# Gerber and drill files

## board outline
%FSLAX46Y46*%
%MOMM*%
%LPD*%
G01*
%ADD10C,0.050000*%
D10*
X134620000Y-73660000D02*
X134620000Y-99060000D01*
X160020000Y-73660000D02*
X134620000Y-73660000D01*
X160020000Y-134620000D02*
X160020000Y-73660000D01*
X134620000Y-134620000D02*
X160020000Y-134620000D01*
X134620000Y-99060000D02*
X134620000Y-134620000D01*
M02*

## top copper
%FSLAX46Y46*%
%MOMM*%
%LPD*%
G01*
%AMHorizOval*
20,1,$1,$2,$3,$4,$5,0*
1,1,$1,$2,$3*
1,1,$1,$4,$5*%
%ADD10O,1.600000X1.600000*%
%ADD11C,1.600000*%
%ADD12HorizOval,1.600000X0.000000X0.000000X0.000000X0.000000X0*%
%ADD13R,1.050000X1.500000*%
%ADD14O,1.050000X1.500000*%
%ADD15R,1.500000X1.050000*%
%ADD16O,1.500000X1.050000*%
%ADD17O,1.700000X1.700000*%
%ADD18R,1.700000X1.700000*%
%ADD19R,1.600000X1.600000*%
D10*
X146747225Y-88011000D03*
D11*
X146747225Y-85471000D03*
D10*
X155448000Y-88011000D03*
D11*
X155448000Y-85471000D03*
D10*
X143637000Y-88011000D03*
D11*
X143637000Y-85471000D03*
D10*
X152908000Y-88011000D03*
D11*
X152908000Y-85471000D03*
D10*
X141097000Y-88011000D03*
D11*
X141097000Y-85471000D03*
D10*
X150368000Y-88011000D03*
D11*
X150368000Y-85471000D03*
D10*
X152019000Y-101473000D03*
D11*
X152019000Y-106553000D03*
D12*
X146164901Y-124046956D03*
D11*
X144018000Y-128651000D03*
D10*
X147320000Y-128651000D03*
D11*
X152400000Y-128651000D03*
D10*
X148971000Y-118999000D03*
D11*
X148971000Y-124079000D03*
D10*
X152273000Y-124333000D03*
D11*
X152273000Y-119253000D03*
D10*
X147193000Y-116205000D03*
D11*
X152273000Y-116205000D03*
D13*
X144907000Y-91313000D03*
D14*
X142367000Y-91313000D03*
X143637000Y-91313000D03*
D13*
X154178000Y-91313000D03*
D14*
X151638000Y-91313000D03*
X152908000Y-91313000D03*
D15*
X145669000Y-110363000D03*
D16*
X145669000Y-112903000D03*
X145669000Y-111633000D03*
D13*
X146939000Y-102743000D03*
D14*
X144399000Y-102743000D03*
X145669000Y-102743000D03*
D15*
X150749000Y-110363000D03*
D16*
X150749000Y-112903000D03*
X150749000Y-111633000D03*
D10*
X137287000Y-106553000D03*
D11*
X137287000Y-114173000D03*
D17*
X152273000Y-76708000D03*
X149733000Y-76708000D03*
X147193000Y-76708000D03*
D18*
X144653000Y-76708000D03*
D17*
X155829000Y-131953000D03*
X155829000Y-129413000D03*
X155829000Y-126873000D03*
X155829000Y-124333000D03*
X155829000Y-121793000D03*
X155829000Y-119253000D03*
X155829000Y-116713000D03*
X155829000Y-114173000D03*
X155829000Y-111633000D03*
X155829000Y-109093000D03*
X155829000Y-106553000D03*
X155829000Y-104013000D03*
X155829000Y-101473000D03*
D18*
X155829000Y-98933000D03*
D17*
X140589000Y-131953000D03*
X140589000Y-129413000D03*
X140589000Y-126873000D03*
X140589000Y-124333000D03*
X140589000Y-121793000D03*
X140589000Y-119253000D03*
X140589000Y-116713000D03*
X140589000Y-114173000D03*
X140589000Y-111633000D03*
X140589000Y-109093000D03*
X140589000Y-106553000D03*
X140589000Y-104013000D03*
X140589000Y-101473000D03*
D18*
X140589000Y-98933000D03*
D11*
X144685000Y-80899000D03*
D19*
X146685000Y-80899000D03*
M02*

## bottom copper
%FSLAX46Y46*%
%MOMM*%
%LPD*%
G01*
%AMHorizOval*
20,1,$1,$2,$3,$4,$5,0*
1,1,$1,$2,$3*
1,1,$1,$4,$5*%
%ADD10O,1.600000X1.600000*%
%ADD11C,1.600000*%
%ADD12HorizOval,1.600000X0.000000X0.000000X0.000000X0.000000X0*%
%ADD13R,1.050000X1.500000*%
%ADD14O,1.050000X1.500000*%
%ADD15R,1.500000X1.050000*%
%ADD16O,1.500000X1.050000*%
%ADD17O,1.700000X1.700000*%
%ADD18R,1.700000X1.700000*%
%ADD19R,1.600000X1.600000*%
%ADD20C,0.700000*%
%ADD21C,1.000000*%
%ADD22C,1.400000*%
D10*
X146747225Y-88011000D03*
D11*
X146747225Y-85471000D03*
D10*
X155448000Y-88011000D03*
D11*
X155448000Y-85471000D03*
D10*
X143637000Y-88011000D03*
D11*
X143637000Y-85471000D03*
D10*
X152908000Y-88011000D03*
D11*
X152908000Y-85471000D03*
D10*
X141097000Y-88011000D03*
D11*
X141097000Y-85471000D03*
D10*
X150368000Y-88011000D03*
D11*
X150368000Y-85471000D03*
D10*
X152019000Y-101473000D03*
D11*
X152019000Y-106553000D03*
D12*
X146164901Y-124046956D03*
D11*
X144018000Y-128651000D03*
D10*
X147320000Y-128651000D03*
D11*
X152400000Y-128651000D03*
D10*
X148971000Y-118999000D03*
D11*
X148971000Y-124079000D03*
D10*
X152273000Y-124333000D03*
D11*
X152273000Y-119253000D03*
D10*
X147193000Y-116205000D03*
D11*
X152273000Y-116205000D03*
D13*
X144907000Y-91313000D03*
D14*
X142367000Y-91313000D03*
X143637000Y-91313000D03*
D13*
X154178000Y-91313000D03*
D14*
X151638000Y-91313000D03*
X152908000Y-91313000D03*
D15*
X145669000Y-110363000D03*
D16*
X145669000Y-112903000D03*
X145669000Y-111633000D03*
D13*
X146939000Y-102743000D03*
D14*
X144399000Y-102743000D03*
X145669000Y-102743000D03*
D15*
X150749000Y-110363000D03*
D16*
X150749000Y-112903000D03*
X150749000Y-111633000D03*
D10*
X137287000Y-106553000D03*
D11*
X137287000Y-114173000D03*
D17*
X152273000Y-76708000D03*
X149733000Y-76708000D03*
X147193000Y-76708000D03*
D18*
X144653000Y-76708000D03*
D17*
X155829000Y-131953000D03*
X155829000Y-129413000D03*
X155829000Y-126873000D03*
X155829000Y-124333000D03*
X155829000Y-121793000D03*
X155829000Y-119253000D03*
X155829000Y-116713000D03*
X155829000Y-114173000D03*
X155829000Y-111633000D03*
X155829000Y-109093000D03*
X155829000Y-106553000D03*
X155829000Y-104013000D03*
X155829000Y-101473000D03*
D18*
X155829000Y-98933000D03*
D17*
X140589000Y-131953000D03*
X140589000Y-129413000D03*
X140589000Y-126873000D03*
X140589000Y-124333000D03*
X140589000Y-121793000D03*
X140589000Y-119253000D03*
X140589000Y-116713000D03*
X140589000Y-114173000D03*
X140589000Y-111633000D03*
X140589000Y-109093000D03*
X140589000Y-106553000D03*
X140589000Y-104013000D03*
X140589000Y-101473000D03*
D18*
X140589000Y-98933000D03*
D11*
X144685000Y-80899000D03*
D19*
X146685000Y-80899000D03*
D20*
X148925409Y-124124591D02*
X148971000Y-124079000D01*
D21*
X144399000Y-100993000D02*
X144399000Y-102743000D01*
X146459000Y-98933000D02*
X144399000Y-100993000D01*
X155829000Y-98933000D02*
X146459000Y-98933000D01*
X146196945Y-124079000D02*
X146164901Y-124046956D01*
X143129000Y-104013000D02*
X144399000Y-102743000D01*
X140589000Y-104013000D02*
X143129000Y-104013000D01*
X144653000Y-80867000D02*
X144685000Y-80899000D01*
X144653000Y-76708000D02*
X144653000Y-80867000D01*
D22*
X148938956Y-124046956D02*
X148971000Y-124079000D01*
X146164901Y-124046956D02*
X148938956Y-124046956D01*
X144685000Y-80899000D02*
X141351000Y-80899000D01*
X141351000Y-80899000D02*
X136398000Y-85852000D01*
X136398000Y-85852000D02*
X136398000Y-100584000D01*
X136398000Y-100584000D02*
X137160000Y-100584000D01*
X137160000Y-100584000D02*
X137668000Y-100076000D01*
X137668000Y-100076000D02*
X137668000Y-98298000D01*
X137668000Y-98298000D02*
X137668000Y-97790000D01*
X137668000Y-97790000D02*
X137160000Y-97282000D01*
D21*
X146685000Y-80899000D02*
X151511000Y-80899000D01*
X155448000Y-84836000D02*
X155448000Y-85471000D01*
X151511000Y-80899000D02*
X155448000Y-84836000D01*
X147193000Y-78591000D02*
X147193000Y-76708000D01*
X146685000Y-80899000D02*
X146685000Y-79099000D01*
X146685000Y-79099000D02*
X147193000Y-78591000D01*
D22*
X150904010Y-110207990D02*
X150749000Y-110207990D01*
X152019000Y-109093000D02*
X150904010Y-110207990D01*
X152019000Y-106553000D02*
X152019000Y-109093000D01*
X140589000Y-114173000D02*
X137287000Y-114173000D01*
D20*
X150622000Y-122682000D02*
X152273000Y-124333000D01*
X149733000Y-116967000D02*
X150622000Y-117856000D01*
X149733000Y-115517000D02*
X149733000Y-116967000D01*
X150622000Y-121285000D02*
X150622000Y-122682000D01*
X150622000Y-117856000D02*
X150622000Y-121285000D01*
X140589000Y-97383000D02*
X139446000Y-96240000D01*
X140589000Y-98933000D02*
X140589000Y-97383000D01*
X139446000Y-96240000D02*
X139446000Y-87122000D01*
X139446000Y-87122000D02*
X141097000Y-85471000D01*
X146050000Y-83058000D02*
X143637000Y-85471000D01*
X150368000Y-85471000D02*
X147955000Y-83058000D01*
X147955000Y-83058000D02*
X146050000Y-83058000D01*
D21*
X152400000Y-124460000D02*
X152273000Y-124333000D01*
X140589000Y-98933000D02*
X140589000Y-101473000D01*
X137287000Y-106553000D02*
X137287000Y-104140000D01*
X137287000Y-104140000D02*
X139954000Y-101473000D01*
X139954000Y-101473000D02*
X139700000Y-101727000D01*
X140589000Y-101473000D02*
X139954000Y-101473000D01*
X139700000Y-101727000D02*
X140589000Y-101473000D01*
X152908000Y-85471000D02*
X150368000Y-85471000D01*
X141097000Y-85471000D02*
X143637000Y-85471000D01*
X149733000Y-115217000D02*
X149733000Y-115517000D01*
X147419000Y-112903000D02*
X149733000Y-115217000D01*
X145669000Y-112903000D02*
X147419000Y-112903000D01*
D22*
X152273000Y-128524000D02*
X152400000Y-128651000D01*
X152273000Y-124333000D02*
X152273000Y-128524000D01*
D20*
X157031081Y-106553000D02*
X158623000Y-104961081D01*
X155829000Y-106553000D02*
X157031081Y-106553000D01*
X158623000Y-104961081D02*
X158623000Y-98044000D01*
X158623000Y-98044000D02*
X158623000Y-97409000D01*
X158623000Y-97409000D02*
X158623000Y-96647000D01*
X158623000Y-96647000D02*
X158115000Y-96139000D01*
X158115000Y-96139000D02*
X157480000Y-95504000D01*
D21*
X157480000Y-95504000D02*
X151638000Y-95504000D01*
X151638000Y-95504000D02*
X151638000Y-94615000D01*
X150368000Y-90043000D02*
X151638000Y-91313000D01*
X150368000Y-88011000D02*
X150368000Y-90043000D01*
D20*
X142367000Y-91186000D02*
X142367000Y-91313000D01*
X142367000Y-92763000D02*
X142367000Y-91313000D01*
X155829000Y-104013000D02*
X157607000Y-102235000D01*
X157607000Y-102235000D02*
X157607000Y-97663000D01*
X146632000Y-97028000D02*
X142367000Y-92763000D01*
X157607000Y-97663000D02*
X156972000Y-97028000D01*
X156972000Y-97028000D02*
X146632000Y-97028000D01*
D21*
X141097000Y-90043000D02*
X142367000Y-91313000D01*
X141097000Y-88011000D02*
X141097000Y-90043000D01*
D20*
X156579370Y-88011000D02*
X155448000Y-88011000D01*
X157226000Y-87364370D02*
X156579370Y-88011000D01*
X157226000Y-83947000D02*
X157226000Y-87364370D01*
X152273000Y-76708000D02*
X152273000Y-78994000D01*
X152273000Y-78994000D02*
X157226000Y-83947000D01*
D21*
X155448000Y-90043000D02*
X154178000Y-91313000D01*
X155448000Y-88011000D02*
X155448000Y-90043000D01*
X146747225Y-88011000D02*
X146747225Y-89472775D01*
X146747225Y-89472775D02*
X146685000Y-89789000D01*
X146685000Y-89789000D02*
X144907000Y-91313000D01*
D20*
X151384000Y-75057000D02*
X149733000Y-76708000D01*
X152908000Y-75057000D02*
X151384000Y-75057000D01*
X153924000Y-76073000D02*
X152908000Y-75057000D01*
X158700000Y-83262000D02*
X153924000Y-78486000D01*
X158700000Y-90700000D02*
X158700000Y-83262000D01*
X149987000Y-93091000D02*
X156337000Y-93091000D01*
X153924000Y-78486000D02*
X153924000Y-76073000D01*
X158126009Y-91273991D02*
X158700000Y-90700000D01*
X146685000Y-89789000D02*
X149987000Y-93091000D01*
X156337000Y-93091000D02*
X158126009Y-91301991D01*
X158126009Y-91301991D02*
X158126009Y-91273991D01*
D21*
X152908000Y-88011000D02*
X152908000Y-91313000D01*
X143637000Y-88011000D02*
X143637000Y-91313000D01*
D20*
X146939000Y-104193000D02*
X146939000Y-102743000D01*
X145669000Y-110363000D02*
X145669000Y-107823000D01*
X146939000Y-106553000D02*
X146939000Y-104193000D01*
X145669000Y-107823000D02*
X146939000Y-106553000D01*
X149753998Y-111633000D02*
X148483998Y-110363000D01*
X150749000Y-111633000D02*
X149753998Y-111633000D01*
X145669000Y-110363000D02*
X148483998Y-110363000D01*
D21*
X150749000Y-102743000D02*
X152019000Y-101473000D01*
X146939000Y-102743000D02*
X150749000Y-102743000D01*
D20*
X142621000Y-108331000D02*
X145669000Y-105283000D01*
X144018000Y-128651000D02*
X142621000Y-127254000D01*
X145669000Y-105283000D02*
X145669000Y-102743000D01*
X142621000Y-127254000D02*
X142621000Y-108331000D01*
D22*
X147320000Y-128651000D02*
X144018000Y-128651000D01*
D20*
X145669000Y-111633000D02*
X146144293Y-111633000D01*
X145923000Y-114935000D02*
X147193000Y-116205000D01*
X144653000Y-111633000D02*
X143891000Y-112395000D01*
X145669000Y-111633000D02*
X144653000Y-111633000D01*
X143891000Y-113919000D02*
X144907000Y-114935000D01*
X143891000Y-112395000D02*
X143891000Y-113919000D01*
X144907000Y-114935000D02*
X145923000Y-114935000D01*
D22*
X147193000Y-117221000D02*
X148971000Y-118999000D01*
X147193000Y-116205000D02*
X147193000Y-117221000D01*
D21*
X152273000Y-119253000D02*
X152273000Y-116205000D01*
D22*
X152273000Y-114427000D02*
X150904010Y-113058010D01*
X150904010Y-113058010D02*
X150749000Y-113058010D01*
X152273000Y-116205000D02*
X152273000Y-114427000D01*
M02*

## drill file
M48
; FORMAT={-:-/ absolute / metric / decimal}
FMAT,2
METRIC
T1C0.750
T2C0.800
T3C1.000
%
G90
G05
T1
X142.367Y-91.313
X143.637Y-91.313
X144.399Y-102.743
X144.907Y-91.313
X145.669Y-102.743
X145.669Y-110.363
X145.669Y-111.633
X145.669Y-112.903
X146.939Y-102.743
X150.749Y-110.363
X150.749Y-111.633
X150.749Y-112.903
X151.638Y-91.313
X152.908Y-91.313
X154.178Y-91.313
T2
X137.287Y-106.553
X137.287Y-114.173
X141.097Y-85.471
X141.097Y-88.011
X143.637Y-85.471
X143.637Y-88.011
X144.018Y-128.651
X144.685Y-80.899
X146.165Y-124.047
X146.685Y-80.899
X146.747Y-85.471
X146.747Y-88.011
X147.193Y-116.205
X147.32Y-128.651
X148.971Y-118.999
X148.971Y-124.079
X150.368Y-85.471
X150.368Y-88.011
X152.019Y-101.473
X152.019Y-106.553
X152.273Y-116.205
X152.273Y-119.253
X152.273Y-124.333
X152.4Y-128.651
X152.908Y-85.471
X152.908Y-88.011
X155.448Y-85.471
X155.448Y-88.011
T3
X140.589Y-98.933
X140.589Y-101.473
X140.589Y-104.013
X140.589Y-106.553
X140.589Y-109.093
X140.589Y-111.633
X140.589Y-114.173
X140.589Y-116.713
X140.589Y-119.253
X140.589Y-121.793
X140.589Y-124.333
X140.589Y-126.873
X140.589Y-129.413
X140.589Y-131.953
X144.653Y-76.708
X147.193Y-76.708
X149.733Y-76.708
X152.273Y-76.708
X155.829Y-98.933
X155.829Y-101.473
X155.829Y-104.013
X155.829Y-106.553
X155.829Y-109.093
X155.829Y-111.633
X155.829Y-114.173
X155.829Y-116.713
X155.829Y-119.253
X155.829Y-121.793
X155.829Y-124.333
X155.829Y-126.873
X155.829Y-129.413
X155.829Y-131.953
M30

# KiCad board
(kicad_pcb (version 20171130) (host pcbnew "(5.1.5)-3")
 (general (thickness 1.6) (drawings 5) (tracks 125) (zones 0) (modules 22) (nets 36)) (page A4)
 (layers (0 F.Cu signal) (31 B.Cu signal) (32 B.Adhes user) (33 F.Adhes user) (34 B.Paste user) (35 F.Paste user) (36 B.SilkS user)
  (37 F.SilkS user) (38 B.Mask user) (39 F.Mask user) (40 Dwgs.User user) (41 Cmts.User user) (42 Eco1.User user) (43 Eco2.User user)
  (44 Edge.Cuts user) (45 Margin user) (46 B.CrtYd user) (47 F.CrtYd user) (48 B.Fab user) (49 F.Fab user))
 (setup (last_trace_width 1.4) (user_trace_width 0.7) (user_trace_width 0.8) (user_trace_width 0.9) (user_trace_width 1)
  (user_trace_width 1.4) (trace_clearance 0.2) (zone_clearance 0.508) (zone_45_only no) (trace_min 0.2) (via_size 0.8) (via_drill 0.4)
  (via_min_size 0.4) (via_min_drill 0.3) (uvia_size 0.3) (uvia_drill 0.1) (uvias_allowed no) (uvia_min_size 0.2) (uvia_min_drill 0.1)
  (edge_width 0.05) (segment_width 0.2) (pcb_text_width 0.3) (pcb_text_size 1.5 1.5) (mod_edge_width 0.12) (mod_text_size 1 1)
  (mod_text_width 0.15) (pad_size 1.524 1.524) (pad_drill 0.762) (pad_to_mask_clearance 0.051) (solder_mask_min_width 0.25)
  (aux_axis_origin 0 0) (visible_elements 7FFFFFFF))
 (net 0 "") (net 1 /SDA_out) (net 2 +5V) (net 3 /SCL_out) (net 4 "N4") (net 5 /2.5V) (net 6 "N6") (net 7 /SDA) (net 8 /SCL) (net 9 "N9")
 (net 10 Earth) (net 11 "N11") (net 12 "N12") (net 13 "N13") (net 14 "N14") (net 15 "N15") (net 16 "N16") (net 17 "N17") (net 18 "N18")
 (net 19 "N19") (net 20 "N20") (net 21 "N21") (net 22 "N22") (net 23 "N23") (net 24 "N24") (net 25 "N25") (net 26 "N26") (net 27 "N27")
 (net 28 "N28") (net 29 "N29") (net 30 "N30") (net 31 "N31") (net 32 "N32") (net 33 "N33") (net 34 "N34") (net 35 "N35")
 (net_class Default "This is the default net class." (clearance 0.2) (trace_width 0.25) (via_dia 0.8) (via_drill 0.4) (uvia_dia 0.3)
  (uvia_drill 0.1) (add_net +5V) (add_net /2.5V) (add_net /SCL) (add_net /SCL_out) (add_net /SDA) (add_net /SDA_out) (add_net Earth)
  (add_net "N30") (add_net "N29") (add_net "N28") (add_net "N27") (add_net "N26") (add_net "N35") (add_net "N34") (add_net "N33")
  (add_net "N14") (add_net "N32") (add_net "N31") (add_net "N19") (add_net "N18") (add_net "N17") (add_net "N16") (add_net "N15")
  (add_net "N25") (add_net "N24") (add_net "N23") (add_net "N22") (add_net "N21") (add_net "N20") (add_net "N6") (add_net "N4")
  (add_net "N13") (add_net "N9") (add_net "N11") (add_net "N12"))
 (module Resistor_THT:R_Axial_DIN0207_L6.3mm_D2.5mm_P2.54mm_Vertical (layer F.Cu) (at 146.747225 85.471 270)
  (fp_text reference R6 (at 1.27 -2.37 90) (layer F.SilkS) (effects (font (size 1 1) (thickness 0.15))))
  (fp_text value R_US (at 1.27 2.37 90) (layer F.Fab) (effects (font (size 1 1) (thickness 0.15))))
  (pad 2 thru_hole oval (at 2.54 0 270) (size 1.6 1.6) (drill 0.8) (layers *.Cu *.Mask) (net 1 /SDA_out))
  (pad 1 thru_hole circle (at 0 0 270) (size 1.6 1.6) (drill 0.8) (layers *.Cu *.Mask) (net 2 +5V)))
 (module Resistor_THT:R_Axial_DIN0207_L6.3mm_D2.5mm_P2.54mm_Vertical (layer F.Cu) (at 155.448 85.471 270)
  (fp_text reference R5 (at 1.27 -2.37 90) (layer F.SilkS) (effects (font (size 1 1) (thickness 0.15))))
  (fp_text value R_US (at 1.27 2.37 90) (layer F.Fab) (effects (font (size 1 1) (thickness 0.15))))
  (pad 2 thru_hole oval (at 2.54 0 270) (size 1.6 1.6) (drill 0.8) (layers *.Cu *.Mask) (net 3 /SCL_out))
  (pad 1 thru_hole circle (at 0 0 270) (size 1.6 1.6) (drill 0.8) (layers *.Cu *.Mask) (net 2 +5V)))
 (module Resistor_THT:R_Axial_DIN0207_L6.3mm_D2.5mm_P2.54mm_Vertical (layer F.Cu) (at 143.637 85.471 270)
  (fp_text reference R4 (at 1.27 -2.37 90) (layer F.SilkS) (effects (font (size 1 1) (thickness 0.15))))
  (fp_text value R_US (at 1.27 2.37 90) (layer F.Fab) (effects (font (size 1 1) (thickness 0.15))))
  (pad 2 thru_hole oval (at 2.54 0 270) (size 1.6 1.6) (drill 0.8) (layers *.Cu *.Mask) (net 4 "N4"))
  (pad 1 thru_hole circle (at 0 0 270) (size 1.6 1.6) (drill 0.8) (layers *.Cu *.Mask) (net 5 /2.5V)))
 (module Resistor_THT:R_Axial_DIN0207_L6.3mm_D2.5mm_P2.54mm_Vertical (layer F.Cu) (at 152.908 85.471 270)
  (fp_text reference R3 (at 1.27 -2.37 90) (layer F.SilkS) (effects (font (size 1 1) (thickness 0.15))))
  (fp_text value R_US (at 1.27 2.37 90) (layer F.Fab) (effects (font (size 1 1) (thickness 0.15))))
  (pad 2 thru_hole oval (at 2.54 0 270) (size 1.6 1.6) (drill 0.8) (layers *.Cu *.Mask) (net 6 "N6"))
  (pad 1 thru_hole circle (at 0 0 270) (size 1.6 1.6) (drill 0.8) (layers *.Cu *.Mask) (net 5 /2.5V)))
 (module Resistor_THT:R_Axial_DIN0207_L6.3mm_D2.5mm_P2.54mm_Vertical (layer F.Cu) (at 141.097 85.471 270)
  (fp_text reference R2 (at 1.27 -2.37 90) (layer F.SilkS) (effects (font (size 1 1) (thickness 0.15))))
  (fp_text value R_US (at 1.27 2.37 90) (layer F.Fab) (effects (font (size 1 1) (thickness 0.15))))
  (pad 2 thru_hole oval (at 2.54 0 270) (size 1.6 1.6) (drill 0.8) (layers *.Cu *.Mask) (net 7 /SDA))
  (pad 1 thru_hole circle (at 0 0 270) (size 1.6 1.6) (drill 0.8) (layers *.Cu *.Mask) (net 5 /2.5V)))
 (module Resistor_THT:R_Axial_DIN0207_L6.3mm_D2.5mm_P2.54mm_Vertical (layer F.Cu) (at 150.368 85.471 270)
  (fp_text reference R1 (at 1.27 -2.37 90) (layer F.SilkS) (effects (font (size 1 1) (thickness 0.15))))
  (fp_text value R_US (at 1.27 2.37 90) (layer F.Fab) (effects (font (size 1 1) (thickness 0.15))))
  (pad 2 thru_hole oval (at 2.54 0 270) (size 1.6 1.6) (drill 0.8) (layers *.Cu *.Mask) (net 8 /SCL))
  (pad 1 thru_hole circle (at 0 0 270) (size 1.6 1.6) (drill 0.8) (layers *.Cu *.Mask) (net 5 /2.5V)))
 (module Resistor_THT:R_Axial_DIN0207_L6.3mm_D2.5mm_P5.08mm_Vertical (layer F.Cu) (at 152.019 106.553 90)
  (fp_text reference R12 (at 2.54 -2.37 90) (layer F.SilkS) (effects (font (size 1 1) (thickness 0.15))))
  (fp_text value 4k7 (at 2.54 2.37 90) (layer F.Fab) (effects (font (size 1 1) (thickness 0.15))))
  (pad 2 thru_hole oval (at 5.08 0 90) (size 1.6 1.6) (drill 0.8) (layers *.Cu *.Mask) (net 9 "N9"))
  (pad 1 thru_hole circle (at 0 0 90) (size 1.6 1.6) (drill 0.8) (layers *.Cu *.Mask) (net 2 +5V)))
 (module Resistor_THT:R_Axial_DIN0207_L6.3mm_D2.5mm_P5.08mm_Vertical (layer F.Cu) (at 144.018 128.651 65)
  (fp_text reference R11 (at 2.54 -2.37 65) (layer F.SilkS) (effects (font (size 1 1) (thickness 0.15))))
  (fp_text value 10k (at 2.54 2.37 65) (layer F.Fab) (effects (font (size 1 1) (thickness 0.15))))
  (pad 2 thru_hole oval (at 5.08 0 65) (size 1.6 1.6) (drill 0.8) (layers *.Cu *.Mask) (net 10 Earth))
  (pad 1 thru_hole circle (at 0 0 65) (size 1.6 1.6) (drill 0.8) (layers *.Cu *.Mask) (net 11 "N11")))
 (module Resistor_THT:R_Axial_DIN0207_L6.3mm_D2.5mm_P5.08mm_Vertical (layer F.Cu) (at 152.4 128.651 180)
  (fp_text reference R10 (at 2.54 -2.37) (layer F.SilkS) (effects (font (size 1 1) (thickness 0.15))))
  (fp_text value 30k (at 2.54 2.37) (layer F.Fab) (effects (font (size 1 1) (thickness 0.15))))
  (pad 2 thru_hole oval (at 5.08 0 180) (size 1.6 1.6) (drill 0.8) (layers *.Cu *.Mask) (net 11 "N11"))
  (pad 1 thru_hole circle (at 0 0 180) (size 1.6 1.6) (drill 0.8) (layers *.Cu *.Mask) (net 5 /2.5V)))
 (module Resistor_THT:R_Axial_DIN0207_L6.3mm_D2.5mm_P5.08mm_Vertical (layer F.Cu) (at 148.971 124.079 90)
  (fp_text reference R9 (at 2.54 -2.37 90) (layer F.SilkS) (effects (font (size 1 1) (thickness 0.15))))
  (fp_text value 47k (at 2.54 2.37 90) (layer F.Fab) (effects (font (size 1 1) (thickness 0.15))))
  (pad 2 thru_hole oval (at 5.08 0 90) (size 1.6 1.6) (drill 0.8) (layers *.Cu *.Mask) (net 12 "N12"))
  (pad 1 thru_hole circle (at 0 0 90) (size 1.6 1.6) (drill 0.8) (layers *.Cu *.Mask) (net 10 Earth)))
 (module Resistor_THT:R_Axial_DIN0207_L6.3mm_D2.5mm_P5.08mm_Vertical (layer F.Cu) (at 152.273 119.253 270)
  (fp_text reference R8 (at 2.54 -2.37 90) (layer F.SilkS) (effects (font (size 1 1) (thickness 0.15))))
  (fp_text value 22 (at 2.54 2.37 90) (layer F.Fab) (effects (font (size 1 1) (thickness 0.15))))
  (pad 2 thru_hole oval (at 5.08 0 270) (size 1.6 1.6) (drill 0.8) (layers *.Cu *.Mask) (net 5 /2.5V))
  (pad 1 thru_hole circle (at 0 0 270) (size 1.6 1.6) (drill 0.8) (layers *.Cu *.Mask) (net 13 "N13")))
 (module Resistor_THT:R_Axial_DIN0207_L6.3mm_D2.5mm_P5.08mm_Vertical (layer F.Cu) (at 152.273 116.205 180)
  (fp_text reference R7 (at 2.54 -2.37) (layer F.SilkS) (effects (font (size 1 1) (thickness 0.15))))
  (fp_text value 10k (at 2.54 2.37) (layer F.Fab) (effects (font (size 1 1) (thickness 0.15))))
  (pad 2 thru_hole oval (at 5.08 0 180) (size 1.6 1.6) (drill 0.8) (layers *.Cu *.Mask) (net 12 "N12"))
  (pad 1 thru_hole circle (at 0 0 180) (size 1.6 1.6) (drill 0.8) (layers *.Cu *.Mask) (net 13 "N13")))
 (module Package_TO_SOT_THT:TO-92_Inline (layer F.Cu) (at 144.907 91.313 180)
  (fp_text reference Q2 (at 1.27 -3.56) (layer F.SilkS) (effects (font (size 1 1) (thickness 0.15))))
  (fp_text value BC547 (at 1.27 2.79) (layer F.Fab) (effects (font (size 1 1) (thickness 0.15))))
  (pad 3 thru_hole rect (at 0 0 180) (size 1.05 1.5) (drill 0.75) (layers *.Cu *.Mask) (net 1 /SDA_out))
  (pad 1 thru_hole oval (at 2.54 0 180) (size 1.05 1.5) (drill 0.75) (layers *.Cu *.Mask) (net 7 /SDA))
  (pad 2 thru_hole oval (at 1.27 0 180) (size 1.05 1.5) (drill 0.75) (layers *.Cu *.Mask) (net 4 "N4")))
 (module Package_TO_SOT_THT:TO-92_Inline (layer F.Cu) (at 154.178 91.313 180)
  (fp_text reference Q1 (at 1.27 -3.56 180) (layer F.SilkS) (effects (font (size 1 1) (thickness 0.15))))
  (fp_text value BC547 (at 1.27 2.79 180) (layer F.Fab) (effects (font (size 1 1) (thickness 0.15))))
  (pad 3 thru_hole rect (at 0 0 180) (size 1.05 1.5) (drill 0.75) (layers *.Cu *.Mask) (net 3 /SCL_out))
  (pad 1 thru_hole oval (at 2.54 0 180) (size 1.05 1.5) (drill 0.75) (layers *.Cu *.Mask) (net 8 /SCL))
  (pad 2 thru_hole oval (at 1.27 0 180) (size 1.05 1.5) (drill 0.75) (layers *.Cu *.Mask) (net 6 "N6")))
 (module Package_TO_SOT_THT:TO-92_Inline (layer F.Cu) (at 145.669 110.363 270)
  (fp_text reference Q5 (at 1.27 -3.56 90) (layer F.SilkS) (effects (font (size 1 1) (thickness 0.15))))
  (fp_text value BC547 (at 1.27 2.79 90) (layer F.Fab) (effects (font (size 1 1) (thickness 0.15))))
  (pad 3 thru_hole rect (at 0 0 270) (size 1.05 1.5) (drill 0.75) (layers *.Cu *.Mask) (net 9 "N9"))
  (pad 1 thru_hole oval (at 2.54 0 270) (size 1.05 1.5) (drill 0.75) (layers *.Cu *.Mask) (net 5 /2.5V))
  (pad 2 thru_hole oval (at 1.27 0 270) (size 1.05 1.5) (drill 0.75) (layers *.Cu *.Mask) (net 12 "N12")))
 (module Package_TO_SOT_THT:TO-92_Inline (layer F.Cu) (at 146.939 102.743 180)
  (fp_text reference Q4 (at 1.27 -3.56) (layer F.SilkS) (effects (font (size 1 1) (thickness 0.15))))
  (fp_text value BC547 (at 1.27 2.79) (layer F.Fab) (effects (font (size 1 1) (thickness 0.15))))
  (pad 3 thru_hole rect (at 0 0 180) (size 1.05 1.5) (drill 0.75) (layers *.Cu *.Mask) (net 9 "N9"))
  (pad 1 thru_hole oval (at 2.54 0 180) (size 1.05 1.5) (drill 0.75) (layers *.Cu *.Mask) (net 10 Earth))
  (pad 2 thru_hole oval (at 1.27 0 180) (size 1.05 1.5) (drill 0.75) (layers *.Cu *.Mask) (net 11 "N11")))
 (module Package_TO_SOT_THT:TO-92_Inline (layer F.Cu) (at 150.749 110.363 270)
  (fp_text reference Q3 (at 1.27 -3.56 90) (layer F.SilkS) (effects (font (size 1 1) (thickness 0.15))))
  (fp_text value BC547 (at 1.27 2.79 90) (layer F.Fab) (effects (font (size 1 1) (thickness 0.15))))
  (pad 3 thru_hole rect (at 0 0 270) (size 1.05 1.5) (drill 0.75) (layers *.Cu *.Mask) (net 2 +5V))
  (pad 1 thru_hole oval (at 2.54 0 270) (size 1.05 1.5) (drill 0.75) (layers *.Cu *.Mask) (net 13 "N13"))
  (pad 2 thru_hole oval (at 1.27 0 270) (size 1.05 1.5) (drill 0.75) (layers *.Cu *.Mask) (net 9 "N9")))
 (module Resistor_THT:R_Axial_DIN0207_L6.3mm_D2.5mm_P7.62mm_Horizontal (layer F.Cu) (at 137.287 114.173 90)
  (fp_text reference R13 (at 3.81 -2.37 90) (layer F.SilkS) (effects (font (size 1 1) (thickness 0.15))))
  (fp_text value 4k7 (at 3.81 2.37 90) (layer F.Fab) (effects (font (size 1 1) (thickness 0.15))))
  (pad 2 thru_hole oval (at 7.62 0 90) (size 1.6 1.6) (drill 0.8) (layers *.Cu *.Mask) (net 5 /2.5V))
  (pad 1 thru_hole circle (at 0 0 90) (size 1.6 1.6) (drill 0.8) (layers *.Cu *.Mask) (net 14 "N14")))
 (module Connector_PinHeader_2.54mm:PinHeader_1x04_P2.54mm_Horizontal (layer F.Cu) (at 144.653 76.708 90)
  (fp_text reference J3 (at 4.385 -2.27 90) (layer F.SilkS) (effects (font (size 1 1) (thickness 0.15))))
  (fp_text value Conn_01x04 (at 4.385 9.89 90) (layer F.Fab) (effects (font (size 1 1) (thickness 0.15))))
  (pad 4 thru_hole oval (at 0 7.62 90) (size 1.7 1.7) (drill 1) (layers *.Cu *.Mask) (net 3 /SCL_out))
  (pad 3 thru_hole oval (at 0 5.08 90) (size 1.7 1.7) (drill 1) (layers *.Cu *.Mask) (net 1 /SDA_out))
  (pad 2 thru_hole oval (at 0 2.54 90) (size 1.7 1.7) (drill 1) (layers *.Cu *.Mask) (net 2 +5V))
  (pad 1 thru_hole rect (at 0 0 90) (size 1.7 1.7) (drill 1) (layers *.Cu *.Mask) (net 10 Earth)))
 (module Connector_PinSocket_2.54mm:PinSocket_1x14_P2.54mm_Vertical (layer F.Cu) (at 155.829 98.933)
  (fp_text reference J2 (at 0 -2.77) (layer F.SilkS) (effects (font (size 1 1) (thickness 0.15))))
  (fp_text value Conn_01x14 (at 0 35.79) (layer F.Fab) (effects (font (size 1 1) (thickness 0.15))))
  (pad 14 thru_hole oval (at 0 33.02) (size 1.7 1.7) (drill 1) (layers *.Cu *.Mask) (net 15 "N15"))
  (pad 13 thru_hole oval (at 0 30.48) (size 1.7 1.7) (drill 1) (layers *.Cu *.Mask) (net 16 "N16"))
  (pad 12 thru_hole oval (at 0 27.94) (size 1.7 1.7) (drill 1) (layers *.Cu *.Mask) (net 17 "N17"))
  (pad 11 thru_hole oval (at 0 25.4) (size 1.7 1.7) (drill 1) (layers *.Cu *.Mask) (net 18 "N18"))
  (pad 10 thru_hole oval (at 0 22.86) (size 1.7 1.7) (drill 1) (layers *.Cu *.Mask) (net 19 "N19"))
  (pad 9 thru_hole oval (at 0 20.32) (size 1.7 1.7) (drill 1) (layers *.Cu *.Mask) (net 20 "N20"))
  (pad 8 thru_hole oval (at 0 17.78) (size 1.7 1.7) (drill 1) (layers *.Cu *.Mask) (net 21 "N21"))
  (pad 7 thru_hole oval (at 0 15.24) (size 1.7 1.7) (drill 1) (layers *.Cu *.Mask) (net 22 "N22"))
  (pad 6 thru_hole oval (at 0 12.7) (size 1.7 1.7) (drill 1) (layers *.Cu *.Mask) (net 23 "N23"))
  (pad 5 thru_hole oval (at 0 10.16) (size 1.7 1.7) (drill 1) (layers *.Cu *.Mask) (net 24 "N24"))
  (pad 4 thru_hole oval (at 0 7.62) (size 1.7 1.7) (drill 1) (layers *.Cu *.Mask) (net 8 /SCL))
  (pad 3 thru_hole oval (at 0 5.08) (size 1.7 1.7) (drill 1) (layers *.Cu *.Mask) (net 7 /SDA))
  (pad 2 thru_hole oval (at 0 2.54) (size 1.7 1.7) (drill 1) (layers *.Cu *.Mask) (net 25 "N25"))
  (pad 1 thru_hole rect (at 0 0) (size 1.7 1.7) (drill 1) (layers *.Cu *.Mask) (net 10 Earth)))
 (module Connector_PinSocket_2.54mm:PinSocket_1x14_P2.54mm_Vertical (layer F.Cu) (at 140.589 98.933)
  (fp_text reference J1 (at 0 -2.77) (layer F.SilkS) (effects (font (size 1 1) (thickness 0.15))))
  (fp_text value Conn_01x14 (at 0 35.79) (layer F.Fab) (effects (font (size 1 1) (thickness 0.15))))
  (pad 14 thru_hole oval (at 0 33.02) (size 1.7 1.7) (drill 1) (layers *.Cu *.Mask) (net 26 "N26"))
  (pad 13 thru_hole oval (at 0 30.48) (size 1.7 1.7) (drill 1) (layers *.Cu *.Mask) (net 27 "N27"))
  (pad 12 thru_hole oval (at 0 27.94) (size 1.7 1.7) (drill 1) (layers *.Cu *.Mask) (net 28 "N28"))
  (pad 11 thru_hole oval (at 0 25.4) (size 1.7 1.7) (drill 1) (layers *.Cu *.Mask) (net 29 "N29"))
  (pad 10 thru_hole oval (at 0 22.86) (size 1.7 1.7) (drill 1) (layers *.Cu *.Mask) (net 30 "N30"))
  (pad 9 thru_hole oval (at 0 20.32) (size 1.7 1.7) (drill 1) (layers *.Cu *.Mask) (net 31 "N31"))
  (pad 8 thru_hole oval (at 0 17.78) (size 1.7 1.7) (drill 1) (layers *.Cu *.Mask) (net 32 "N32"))
  (pad 7 thru_hole oval (at 0 15.24) (size 1.7 1.7) (drill 1) (layers *.Cu *.Mask) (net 14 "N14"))
  (pad 6 thru_hole oval (at 0 12.7) (size 1.7 1.7) (drill 1) (layers *.Cu *.Mask) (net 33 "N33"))
  (pad 5 thru_hole oval (at 0 10.16) (size 1.7 1.7) (drill 1) (layers *.Cu *.Mask) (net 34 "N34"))
  (pad 4 thru_hole oval (at 0 7.62) (size 1.7 1.7) (drill 1) (layers *.Cu *.Mask) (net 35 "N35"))
  (pad 3 thru_hole oval (at 0 5.08) (size 1.7 1.7) (drill 1) (layers *.Cu *.Mask) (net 10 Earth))
  (pad 2 thru_hole oval (at 0 2.54) (size 1.7 1.7) (drill 1) (layers *.Cu *.Mask) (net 5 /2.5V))
  (pad 1 thru_hole rect (at 0 0) (size 1.7 1.7) (drill 1) (layers *.Cu *.Mask) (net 5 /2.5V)))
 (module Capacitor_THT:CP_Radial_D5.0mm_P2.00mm (layer F.Cu) (at 146.685 80.899 180)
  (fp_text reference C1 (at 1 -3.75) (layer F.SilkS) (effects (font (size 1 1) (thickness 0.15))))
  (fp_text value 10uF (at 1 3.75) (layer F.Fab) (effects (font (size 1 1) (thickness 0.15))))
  (pad 2 thru_hole circle (at 2 0 180) (size 1.6 1.6) (drill 0.8) (layers *.Cu *.Mask) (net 10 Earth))
  (pad 1 thru_hole rect (at 0 0 180) (size 1.6 1.6) (drill 0.8) (layers *.Cu *.Mask) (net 2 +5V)))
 (gr_line (start 134.62 73.66) (end 134.62 99.06) (layer Edge.Cuts) (width 0.05))
 (gr_line (start 160.02 73.66) (end 134.62 73.66) (layer Edge.Cuts) (width 0.05))
 (gr_line (start 160.02 134.62) (end 160.02 73.66) (layer Edge.Cuts) (width 0.05))
 (gr_line (start 134.62 134.62) (end 160.02 134.62) (layer Edge.Cuts) (width 0.05))
 (gr_line (start 134.62 99.06) (end 134.62 134.62) (layer Edge.Cuts) (width 0.05))
 (segment (start 148.925409 124.124591) (end 148.971 124.079) (width 0.7) (layer B.Cu) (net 10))
 (segment (start 144.399 100.993) (end 144.399 102.743) (width 1) (layer B.Cu) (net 10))
 (segment (start 146.459 98.933) (end 144.399 100.993) (width 1) (layer B.Cu) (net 10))
 (segment (start 155.829 98.933) (end 146.459 98.933) (width 1) (layer B.Cu) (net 10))
 (segment (start 146.196945 124.079) (end 146.164901 124.046956) (width 1) (layer B.Cu) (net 10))
 (segment (start 143.129 104.013) (end 144.399 102.743) (width 1) (layer B.Cu) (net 10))
 (segment (start 140.589 104.013) (end 143.129 104.013) (width 1) (layer B.Cu) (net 10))
 (segment (start 144.653 80.867) (end 144.685 80.899) (width 1) (layer B.Cu) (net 10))
 (segment (start 144.653 76.708) (end 144.653 80.867) (width 1) (layer B.Cu) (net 10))
 (segment (start 148.938956 124.046956) (end 148.971 124.079) (width 1.4) (layer B.Cu) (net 10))
 (segment (start 146.164901 124.046956) (end 148.938956 124.046956) (width 1.4) (layer B.Cu) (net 10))
 (segment (start 144.685 80.899) (end 141.351 80.899) (width 1.4) (layer B.Cu) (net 10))
 (segment (start 141.351 80.899) (end 136.398 85.852) (width 1.4) (layer B.Cu) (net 10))
 (segment (start 136.398 85.852) (end 136.398 100.584) (width 1.4) (layer B.Cu) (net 10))
 (segment (start 136.398 100.584) (end 137.16 100.584) (width 1.4) (layer B.Cu) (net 10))
 (segment (start 137.16 100.584) (end 137.668 100.076) (width 1.4) (layer B.Cu) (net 10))
 (segment (start 137.668 100.076) (end 137.668 98.298) (width 1.4) (layer B.Cu) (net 10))
 (segment (start 137.668 98.298) (end 137.668 97.79) (width 1.4) (layer B.Cu) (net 10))
 (segment (start 137.668 97.79) (end 137.16 97.282) (width 1.4) (layer B.Cu) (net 10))
 (segment (start 146.685 80.899) (end 151.511 80.899) (width 1) (layer B.Cu) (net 2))
 (segment (start 155.448 84.836) (end 155.448 85.471) (width 1) (layer B.Cu) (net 2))
 (segment (start 151.511 80.899) (end 155.448 84.836) (width 1) (layer B.Cu) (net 2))
 (segment (start 147.193 78.591) (end 147.193 76.708) (width 1) (layer B.Cu) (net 2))
 (segment (start 146.685 80.899) (end 146.685 79.099) (width 1) (layer B.Cu) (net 2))
 (segment (start 146.685 79.099) (end 147.193 78.591) (width 1) (layer B.Cu) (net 2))
 (segment (start 150.90401 110.20799) (end 150.749 110.20799) (width 1.4) (layer B.Cu) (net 2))
 (segment (start 152.019 109.093) (end 150.90401 110.20799) (width 1.4) (layer B.Cu) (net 2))
 (segment (start 152.019 106.553) (end 152.019 109.093) (width 1.4) (layer B.Cu) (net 2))
 (segment (start 140.589 114.173) (end 137.287 114.173) (width 1.4) (layer B.Cu) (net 14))
 (segment (start 150.622 122.682) (end 152.273 124.333) (width 0.7) (layer B.Cu) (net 5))
 (segment (start 149.733 116.967) (end 150.622 117.856) (width 0.7) (layer B.Cu) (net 5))
 (segment (start 149.733 115.517) (end 149.733 116.967) (width 0.7) (layer B.Cu) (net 5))
 (segment (start 150.622 121.285) (end 150.622 122.682) (width 0.7) (layer B.Cu) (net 5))
 (segment (start 150.622 117.856) (end 150.622 121.285) (width 0.7) (layer B.Cu) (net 5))
 (segment (start 140.589 97.383) (end 139.446 96.24) (width 0.7) (layer B.Cu) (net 5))
 (segment (start 140.589 98.933) (end 140.589 97.383) (width 0.7) (layer B.Cu) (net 5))
 (segment (start 139.446 96.24) (end 139.446 87.122) (width 0.7) (layer B.Cu) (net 5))
 (segment (start 139.446 87.122) (end 141.097 85.471) (width 0.7) (layer B.Cu) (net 5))
 (segment (start 146.05 83.058) (end 143.637 85.471) (width 0.7) (layer B.Cu) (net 5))
 (segment (start 150.368 85.471) (end 147.955 83.058) (width 0.7) (layer B.Cu) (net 5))
 (segment (start 147.955 83.058) (end 146.05 83.058) (width 0.7) (layer B.Cu) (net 5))
 (segment (start 152.4 124.46) (end 152.273 124.333) (width 1) (layer B.Cu) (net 5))
 (segment (start 140.589 98.933) (end 140.589 101.473) (width 1) (layer B.Cu) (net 5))
 (segment (start 137.287 106.553) (end 137.287 104.14) (width 1) (layer B.Cu) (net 5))
 (segment (start 137.287 104.14) (end 139.954 101.473) (width 1) (layer B.Cu) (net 5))
 (segment (start 139.954 101.473) (end 139.7 101.727) (width 1) (layer B.Cu) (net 5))
 (segment (start 140.589 101.473) (end 139.954 101.473) (width 1) (layer B.Cu) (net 5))
 (segment (start 139.7 101.727) (end 140.589 101.473) (width 1) (layer B.Cu) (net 5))
 (segment (start 152.908 85.471) (end 150.368 85.471) (width 1) (layer B.Cu) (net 5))
 (segment (start 141.097 85.471) (end 143.637 85.471) (width 1) (layer B.Cu) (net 5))
 (segment (start 149.733 115.217) (end 149.733 115.517) (width 1) (layer B.Cu) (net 5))
 (segment (start 147.419 112.903) (end 149.733 115.217) (width 1) (layer B.Cu) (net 5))
 (segment (start 145.669 112.903) (end 147.419 112.903) (width 1) (layer B.Cu) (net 5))
 (segment (start 152.273 128.524) (end 152.4 128.651) (width 1.4) (layer B.Cu) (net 5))
 (segment (start 152.273 124.333) (end 152.273 128.524) (width 1.4) (layer B.Cu) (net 5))
 (segment (start 157.031081 106.553) (end 158.623 104.961081) (width 0.7) (layer B.Cu) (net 8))
 (segment (start 155.829 106.553) (end 157.031081 106.553) (width 0.7) (layer B.Cu) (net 8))
 (segment (start 158.623 104.961081) (end 158.623 98.044) (width 0.7) (layer B.Cu) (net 8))
 (segment (start 158.623 98.044) (end 158.623 97.409) (width 0.7) (layer B.Cu) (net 8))
 (segment (start 158.623 97.409) (end 158.623 96.647) (width 0.7) (layer B.Cu) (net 8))
 (segment (start 158.623 96.647) (end 158.115 96.139) (width 0.7) (layer B.Cu) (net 8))
 (segment (start 158.115 96.139) (end 157.48 95.504) (width 0.7) (layer B.Cu) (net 8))
 (segment (start 157.48 95.504) (end 151.638 95.504) (width 1) (layer B.Cu) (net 8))
 (segment (start 151.638 95.504) (end 151.638 94.615) (width 1) (layer B.Cu) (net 8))
 (segment (start 150.368 90.043) (end 151.638 91.313) (width 1) (layer B.Cu) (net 8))
 (segment (start 150.368 88.011) (end 150.368 90.043) (width 1) (layer B.Cu) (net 8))
 (segment (start 142.367 91.186) (end 142.367 91.313) (width 0.7) (layer B.Cu) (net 7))
 (segment (start 142.367 92.763) (end 142.367 91.313) (width 0.7) (layer B.Cu) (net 7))
 (segment (start 155.829 104.013) (end 157.607 102.235) (width 0.7) (layer B.Cu) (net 7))
 (segment (start 157.607 102.235) (end 157.607 97.663) (width 0.7) (layer B.Cu) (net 7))
 (segment (start 146.632 97.028) (end 142.367 92.763) (width 0.7) (layer B.Cu) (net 7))
 (segment (start 157.607 97.663) (end 156.972 97.028) (width 0.7) (layer B.Cu) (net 7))
 (segment (start 156.972 97.028) (end 146.632 97.028) (width 0.7) (layer B.Cu) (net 7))
 (segment (start 141.097 90.043) (end 142.367 91.313) (width 1) (layer B.Cu) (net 7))
 (segment (start 141.097 88.011) (end 141.097 90.043) (width 1) (layer B.Cu) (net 7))
 (segment (start 156.57937 88.011) (end 155.448 88.011) (width 0.7) (layer B.Cu) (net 3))
 (segment (start 157.226 87.36437) (end 156.57937 88.011) (width 0.7) (layer B.Cu) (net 3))
 (segment (start 157.226 83.947) (end 157.226 87.36437) (width 0.7) (layer B.Cu) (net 3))
 (segment (start 152.273 76.708) (end 152.273 78.994) (width 0.7) (layer B.Cu) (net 3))
 (segment (start 152.273 78.994) (end 157.226 83.947) (width 0.7) (layer B.Cu) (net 3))
 (segment (start 155.448 90.043) (end 154.178 91.313) (width 1) (layer B.Cu) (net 3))
 (segment (start 155.448 88.011) (end 155.448 90.043) (width 1) (layer B.Cu) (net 3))
 (segment (start 146.747225 88.011) (end 146.747225 89.472775) (width 1) (layer B.Cu) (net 1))
 (segment (start 146.747225 89.472775) (end 146.685 89.789) (width 1) (layer B.Cu) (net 1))
 (segment (start 146.685 89.789) (end 144.907 91.313) (width 1) (layer B.Cu) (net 1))
 (segment (start 151.384 75.057) (end 149.733 76.708) (width 0.7) (layer B.Cu) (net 1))
 (segment (start 152.908 75.057) (end 151.384 75.057) (width 0.7) (layer B.Cu) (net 1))
 (segment (start 153.924 76.073) (end 152.908 75.057) (width 0.7) (layer B.Cu) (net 1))
 (segment (start 158.7 83.262) (end 153.924 78.486) (width 0.7) (layer B.Cu) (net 1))
 (segment (start 158.7 90.7) (end 158.7 83.262) (width 0.7) (layer B.Cu) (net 1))
 (segment (start 149.987 93.091) (end 156.337 93.091) (width 0.7) (layer B.Cu) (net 1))
 (segment (start 153.924 78.486) (end 153.924 76.073) (width 0.7) (layer B.Cu) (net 1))
 (segment (start 158.126009 91.273991) (end 158.7 90.7) (width 0.7) (layer B.Cu) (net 1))
 (segment (start 146.685 89.789) (end 149.987 93.091) (width 0.7) (layer B.Cu) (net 1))
 (segment (start 156.337 93.091) (end 158.126009 91.301991) (width 0.7) (layer B.Cu) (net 1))
 (segment (start 158.126009 91.301991) (end 158.126009 91.273991) (width 0.7) (layer B.Cu) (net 1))
 (segment (start 152.908 88.011) (end 152.908 91.313) (width 1) (layer B.Cu) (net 6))
 (segment (start 143.637 88.011) (end 143.637 91.313) (width 1) (layer B.Cu) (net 4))
 (segment (start 146.939 104.193) (end 146.939 102.743) (width 0.7) (layer B.Cu) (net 9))
 (segment (start 145.669 110.363) (end 145.669 107.823) (width 0.7) (layer B.Cu) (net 9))
 (segment (start 146.939 106.553) (end 146.939 104.193) (width 0.7) (layer B.Cu) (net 9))
 (segment (start 145.669 107.823) (end 146.939 106.553) (width 0.7) (layer B.Cu) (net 9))
 (segment (start 149.753998 111.633) (end 148.483998 110.363) (width 0.7) (layer B.Cu) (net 9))
 (segment (start 150.749 111.633) (end 149.753998 111.633) (width 0.7) (layer B.Cu) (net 9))
 (segment (start 145.669 110.363) (end 148.483998 110.363) (width 0.7) (layer B.Cu) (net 9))
 (segment (start 150.749 102.743) (end 152.019 101.473) (width 1) (layer B.Cu) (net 9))
 (segment (start 146.939 102.743) (end 150.749 102.743) (width 1) (layer B.Cu) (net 9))
 (segment (start 142.621 108.331) (end 145.669 105.283) (width 0.7) (layer B.Cu) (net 11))
 (segment (start 144.018 128.651) (end 142.621 127.254) (width 0.7) (layer B.Cu) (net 11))
 (segment (start 145.669 105.283) (end 145.669 102.743) (width 0.7) (layer B.Cu) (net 11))
 (segment (start 142.621 127.254) (end 142.621 108.331) (width 0.7) (layer B.Cu) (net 11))
 (segment (start 147.32 128.651) (end 144.018 128.651) (width 1.4) (layer B.Cu) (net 11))
 (segment (start 145.669 111.633) (end 146.144293 111.633) (width 0.7) (layer B.Cu) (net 12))
 (segment (start 145.923 114.935) (end 147.193 116.205) (width 0.7) (layer B.Cu) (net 12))
 (segment (start 144.653 111.633) (end 143.891 112.395) (width 0.7) (layer B.Cu) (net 12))
 (segment (start 145.669 111.633) (end 144.653 111.633) (width 0.7) (layer B.Cu) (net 12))
 (segment (start 143.891 113.919) (end 144.907 114.935) (width 0.7) (layer B.Cu) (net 12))
 (segment (start 143.891 112.395) (end 143.891 113.919) (width 0.7) (layer B.Cu) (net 12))
 (segment (start 144.907 114.935) (end 145.923 114.935) (width 0.7) (layer B.Cu) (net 12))
 (segment (start 147.193 117.221) (end 148.971 118.999) (width 1.4) (layer B.Cu) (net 12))
 (segment (start 147.193 116.205) (end 147.193 117.221) (width 1.4) (layer B.Cu) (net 12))
 (segment (start 152.273 119.253) (end 152.273 116.205) (width 1) (layer B.Cu) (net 13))
 (segment (start 152.273 114.427) (end 150.90401 113.05801) (width 1.4) (layer B.Cu) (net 13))
 (segment (start 150.90401 113.05801) (end 150.749 113.05801) (width 1.4) (layer B.Cu) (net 13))
 (segment (start 152.273 116.205) (end 152.273 114.427) (width 1.4) (layer B.Cu) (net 13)))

